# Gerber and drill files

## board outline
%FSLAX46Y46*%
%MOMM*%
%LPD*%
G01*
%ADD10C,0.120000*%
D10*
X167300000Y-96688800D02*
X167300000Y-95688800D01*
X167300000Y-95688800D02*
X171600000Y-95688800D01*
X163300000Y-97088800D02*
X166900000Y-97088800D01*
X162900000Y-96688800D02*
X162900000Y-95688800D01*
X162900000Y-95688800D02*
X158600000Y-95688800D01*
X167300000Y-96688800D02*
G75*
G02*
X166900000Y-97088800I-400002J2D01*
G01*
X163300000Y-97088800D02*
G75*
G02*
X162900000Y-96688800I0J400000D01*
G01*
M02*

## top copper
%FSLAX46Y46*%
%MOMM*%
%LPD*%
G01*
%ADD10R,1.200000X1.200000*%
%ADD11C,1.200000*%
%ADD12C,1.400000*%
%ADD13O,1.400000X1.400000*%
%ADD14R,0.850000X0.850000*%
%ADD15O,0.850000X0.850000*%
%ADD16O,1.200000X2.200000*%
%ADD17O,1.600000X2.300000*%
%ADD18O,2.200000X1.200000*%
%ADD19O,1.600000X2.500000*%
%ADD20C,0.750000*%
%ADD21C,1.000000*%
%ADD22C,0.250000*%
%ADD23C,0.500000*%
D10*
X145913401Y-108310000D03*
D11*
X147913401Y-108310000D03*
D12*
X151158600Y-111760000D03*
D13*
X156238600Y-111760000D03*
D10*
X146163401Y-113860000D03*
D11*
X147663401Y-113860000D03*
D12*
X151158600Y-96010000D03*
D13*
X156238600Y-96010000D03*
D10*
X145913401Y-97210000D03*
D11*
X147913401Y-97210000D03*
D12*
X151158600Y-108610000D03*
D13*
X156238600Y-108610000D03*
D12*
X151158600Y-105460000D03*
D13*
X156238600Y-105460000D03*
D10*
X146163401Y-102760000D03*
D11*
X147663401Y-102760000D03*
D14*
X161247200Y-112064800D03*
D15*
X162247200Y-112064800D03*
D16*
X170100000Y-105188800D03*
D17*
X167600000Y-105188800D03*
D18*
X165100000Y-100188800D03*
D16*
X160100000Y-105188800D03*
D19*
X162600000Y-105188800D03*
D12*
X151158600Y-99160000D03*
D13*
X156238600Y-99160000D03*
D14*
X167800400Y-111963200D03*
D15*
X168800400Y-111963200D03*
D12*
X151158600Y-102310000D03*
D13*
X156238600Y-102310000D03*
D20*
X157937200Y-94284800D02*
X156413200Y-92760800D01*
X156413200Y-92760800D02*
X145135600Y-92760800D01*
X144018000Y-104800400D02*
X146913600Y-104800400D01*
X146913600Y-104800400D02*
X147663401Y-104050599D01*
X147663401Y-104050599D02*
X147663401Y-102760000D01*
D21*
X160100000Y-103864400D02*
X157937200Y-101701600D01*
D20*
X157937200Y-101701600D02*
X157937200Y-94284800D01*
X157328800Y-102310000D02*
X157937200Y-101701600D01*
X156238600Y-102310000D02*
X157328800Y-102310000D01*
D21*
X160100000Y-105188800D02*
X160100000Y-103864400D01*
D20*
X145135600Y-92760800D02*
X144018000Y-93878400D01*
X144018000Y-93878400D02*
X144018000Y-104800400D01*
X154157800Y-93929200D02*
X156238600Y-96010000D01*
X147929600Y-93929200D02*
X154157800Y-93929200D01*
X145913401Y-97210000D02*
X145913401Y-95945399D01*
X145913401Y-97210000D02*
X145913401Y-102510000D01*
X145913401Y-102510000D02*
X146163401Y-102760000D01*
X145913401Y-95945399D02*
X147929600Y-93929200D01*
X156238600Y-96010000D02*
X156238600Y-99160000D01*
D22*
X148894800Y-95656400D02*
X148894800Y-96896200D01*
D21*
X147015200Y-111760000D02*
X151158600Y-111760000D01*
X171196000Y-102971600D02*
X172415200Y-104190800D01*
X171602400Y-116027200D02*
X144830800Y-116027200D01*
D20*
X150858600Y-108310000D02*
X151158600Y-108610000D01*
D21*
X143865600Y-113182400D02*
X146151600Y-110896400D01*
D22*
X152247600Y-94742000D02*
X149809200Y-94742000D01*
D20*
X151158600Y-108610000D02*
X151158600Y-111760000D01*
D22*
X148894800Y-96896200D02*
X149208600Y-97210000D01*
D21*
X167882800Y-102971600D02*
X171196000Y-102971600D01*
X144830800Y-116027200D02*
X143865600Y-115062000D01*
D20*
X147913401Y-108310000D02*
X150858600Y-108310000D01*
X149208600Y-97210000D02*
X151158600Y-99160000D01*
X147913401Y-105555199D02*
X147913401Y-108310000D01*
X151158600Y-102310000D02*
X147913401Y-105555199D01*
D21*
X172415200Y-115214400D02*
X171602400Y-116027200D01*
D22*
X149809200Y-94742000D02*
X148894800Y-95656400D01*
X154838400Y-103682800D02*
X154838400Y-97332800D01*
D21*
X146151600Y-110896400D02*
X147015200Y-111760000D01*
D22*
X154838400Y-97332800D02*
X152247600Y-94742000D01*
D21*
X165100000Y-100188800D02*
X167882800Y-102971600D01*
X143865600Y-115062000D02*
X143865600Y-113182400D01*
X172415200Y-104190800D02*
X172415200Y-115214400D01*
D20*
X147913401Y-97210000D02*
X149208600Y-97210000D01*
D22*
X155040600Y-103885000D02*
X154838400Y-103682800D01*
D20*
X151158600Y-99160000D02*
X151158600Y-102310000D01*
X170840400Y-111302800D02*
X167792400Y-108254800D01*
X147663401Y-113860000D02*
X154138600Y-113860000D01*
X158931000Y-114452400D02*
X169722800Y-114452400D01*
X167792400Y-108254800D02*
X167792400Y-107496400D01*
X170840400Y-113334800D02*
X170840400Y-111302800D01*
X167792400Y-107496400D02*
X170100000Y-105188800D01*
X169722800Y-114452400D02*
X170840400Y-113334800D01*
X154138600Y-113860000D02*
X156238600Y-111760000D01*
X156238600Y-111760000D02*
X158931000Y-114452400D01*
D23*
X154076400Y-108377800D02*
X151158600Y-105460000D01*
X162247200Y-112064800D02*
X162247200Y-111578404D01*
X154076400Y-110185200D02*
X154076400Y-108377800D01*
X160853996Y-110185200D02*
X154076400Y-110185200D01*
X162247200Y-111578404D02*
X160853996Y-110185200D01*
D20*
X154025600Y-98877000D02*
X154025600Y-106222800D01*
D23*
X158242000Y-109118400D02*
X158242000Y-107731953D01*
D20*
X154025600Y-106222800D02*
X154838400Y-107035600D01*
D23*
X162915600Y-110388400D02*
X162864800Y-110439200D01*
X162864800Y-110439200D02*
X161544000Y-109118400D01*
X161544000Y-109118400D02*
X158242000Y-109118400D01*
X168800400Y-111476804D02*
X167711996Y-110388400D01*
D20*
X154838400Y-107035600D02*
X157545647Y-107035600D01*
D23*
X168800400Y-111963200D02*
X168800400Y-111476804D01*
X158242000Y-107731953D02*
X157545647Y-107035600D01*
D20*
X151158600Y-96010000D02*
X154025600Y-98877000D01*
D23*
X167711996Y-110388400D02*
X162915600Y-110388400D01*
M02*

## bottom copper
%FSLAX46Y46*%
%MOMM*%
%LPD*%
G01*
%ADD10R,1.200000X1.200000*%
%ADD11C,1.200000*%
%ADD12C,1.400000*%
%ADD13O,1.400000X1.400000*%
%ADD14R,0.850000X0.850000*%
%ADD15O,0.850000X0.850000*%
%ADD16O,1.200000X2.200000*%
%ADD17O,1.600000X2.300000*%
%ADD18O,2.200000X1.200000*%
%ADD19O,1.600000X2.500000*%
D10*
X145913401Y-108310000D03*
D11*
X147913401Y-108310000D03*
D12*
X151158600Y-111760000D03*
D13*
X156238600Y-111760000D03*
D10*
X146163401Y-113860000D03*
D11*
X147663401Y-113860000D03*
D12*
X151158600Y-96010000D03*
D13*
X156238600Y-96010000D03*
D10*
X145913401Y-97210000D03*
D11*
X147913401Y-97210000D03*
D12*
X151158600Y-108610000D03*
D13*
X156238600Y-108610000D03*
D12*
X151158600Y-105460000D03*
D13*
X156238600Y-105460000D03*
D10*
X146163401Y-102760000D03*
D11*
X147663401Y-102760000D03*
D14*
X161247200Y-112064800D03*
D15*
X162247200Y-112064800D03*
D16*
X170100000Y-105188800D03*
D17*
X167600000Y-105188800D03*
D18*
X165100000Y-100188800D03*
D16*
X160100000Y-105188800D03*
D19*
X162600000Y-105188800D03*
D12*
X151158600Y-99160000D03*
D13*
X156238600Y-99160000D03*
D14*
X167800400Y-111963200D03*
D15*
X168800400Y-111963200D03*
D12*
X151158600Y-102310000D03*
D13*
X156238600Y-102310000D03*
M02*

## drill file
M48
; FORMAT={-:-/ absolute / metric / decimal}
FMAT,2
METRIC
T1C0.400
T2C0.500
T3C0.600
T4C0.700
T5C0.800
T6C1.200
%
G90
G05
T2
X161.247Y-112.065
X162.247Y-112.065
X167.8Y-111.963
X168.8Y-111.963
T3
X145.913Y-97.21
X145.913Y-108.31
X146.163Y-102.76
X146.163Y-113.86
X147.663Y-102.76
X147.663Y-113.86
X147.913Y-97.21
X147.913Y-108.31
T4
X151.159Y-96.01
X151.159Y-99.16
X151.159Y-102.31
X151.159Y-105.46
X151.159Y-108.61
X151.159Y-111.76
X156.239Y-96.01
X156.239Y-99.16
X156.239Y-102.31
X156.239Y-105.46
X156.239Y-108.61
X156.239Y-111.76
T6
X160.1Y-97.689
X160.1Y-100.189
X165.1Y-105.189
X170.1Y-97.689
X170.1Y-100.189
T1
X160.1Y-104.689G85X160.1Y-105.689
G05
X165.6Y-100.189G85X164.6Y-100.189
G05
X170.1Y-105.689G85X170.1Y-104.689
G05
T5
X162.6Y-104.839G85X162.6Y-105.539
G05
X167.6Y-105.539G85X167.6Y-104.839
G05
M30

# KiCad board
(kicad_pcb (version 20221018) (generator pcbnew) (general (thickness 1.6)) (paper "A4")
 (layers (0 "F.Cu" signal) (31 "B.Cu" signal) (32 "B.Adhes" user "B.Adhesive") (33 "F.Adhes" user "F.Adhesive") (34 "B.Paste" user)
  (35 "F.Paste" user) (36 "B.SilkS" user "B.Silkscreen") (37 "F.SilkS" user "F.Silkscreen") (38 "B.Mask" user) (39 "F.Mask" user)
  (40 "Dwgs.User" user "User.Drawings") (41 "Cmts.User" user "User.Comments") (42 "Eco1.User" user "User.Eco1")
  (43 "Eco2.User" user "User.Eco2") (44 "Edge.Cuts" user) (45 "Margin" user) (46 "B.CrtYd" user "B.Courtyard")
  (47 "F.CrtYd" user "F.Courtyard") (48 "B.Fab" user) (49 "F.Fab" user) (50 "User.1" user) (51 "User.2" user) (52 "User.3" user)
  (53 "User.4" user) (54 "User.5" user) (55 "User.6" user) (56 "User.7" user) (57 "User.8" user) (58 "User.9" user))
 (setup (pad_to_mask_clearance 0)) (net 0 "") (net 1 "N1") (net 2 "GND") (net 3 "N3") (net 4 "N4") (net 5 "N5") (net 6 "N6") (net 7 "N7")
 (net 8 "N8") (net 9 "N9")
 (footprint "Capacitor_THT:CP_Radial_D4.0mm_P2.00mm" (layer "F.Cu") (at 145.913401 108.31)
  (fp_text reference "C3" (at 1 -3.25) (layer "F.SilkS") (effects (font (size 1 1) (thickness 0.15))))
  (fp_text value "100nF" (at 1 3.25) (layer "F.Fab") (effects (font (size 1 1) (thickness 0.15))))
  (pad "1" thru_hole rect (at 0 0) (size 1.2 1.2) (drill 0.6) (layers "*.Cu" "*.Mask") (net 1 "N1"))
  (pad "2" thru_hole circle (at 2 0) (size 1.2 1.2) (drill 0.6) (layers "*.Cu" "*.Mask") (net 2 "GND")))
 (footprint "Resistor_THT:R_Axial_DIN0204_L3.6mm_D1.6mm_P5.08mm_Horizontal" (layer "F.Cu") (at 151.1586 111.76)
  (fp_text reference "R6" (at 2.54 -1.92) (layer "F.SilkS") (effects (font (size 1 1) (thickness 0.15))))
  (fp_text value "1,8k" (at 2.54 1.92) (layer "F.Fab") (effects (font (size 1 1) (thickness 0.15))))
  (pad "1" thru_hole circle (at 0 0) (size 1.4 1.4) (drill 0.7) (layers "*.Cu" "*.Mask") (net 2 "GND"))
  (pad "2" thru_hole oval (at 5.08 0) (size 1.4 1.4) (drill 0.7) (layers "*.Cu" "*.Mask") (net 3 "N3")))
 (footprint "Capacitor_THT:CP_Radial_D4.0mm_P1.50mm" (layer "F.Cu") (at 146.163401 113.86)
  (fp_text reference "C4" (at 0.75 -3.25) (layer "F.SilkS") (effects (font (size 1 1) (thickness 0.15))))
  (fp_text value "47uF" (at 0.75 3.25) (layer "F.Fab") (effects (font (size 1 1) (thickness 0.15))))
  (pad "1" thru_hole rect (at 0 0) (size 1.2 1.2) (drill 0.6) (layers "*.Cu" "*.Mask") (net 1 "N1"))
  (pad "2" thru_hole circle (at 1.5 0) (size 1.2 1.2) (drill 0.6) (layers "*.Cu" "*.Mask") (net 3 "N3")))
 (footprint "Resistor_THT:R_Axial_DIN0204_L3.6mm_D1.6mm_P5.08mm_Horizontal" (layer "F.Cu") (at 151.1586 96.01)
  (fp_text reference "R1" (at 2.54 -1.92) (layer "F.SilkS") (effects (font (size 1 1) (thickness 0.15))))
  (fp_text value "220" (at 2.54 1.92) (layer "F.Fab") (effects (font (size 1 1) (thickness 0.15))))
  (pad "1" thru_hole circle (at 0 0) (size 1.4 1.4) (drill 0.7) (layers "*.Cu" "*.Mask") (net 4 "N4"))
  (pad "2" thru_hole oval (at 5.08 0) (size 1.4 1.4) (drill 0.7) (layers "*.Cu" "*.Mask") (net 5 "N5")))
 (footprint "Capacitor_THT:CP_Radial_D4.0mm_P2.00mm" (layer "F.Cu") (at 145.913401 97.21)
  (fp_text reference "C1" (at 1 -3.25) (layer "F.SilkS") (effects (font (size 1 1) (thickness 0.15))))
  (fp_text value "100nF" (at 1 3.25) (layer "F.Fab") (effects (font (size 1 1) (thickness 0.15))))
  (pad "1" thru_hole rect (at 0 0) (size 1.2 1.2) (drill 0.6) (layers "*.Cu" "*.Mask") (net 5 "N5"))
  (pad "2" thru_hole circle (at 2 0) (size 1.2 1.2) (drill 0.6) (layers "*.Cu" "*.Mask") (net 2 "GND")))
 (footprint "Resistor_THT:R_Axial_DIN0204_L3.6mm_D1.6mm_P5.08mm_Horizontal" (layer "F.Cu") (at 151.1586 108.61)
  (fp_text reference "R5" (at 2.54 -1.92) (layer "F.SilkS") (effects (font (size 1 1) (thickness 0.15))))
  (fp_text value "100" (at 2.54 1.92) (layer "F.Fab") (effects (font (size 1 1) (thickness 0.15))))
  (pad "1" thru_hole circle (at 0 0) (size 1.4 1.4) (drill 0.7) (layers "*.Cu" "*.Mask") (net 2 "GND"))
  (pad "2" thru_hole oval (at 5.08 0) (size 1.4 1.4) (drill 0.7) (layers "*.Cu" "*.Mask") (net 1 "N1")))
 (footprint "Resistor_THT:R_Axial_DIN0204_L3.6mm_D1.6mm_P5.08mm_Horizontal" (layer "F.Cu") (at 151.1586 105.46)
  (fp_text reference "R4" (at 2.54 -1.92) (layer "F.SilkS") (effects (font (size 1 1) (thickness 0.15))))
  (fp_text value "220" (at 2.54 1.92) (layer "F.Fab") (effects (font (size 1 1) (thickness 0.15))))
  (pad "1" thru_hole circle (at 0 0) (size 1.4 1.4) (drill 0.7) (layers "*.Cu" "*.Mask") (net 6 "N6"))
  (pad "2" thru_hole oval (at 5.08 0) (size 1.4 1.4) (drill 0.7) (layers "*.Cu" "*.Mask") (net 1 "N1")))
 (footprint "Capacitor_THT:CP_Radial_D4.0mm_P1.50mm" (layer "F.Cu") (at 146.163401 102.76)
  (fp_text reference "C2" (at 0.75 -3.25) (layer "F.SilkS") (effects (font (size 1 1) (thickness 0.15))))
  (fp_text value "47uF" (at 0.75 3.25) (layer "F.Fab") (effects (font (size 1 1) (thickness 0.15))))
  (pad "1" thru_hole rect (at 0 0) (size 1.2 1.2) (drill 0.6) (layers "*.Cu" "*.Mask") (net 5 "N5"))
  (pad "2" thru_hole circle (at 1.5 0) (size 1.2 1.2) (drill 0.6) (layers "*.Cu" "*.Mask") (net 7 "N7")))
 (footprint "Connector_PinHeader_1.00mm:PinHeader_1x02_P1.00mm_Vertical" (layer "F.Cu") (at 161.2472 112.0648 90)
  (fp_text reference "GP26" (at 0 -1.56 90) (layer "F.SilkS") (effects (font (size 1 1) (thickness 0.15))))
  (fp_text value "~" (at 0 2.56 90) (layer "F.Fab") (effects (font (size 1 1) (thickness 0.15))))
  (pad "1" thru_hole rect (at 0 0 90) (size 0.85 0.85) (drill 0.5) (layers "*.Cu" "*.Mask") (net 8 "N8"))
  (pad "2" thru_hole oval (at 0 1 90) (size 0.85 0.85) (drill 0.5) (layers "*.Cu" "*.Mask") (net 6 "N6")))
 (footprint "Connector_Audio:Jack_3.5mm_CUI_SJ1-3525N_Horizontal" (layer "F.Cu") (at 165.1 100.1888 180)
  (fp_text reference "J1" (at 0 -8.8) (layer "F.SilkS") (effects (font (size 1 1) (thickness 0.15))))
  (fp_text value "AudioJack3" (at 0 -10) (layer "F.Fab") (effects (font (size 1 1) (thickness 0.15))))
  (fp_line (start -2.2 3.5) (end -2.2 4.5) (stroke (width 0.12) (type solid)) (layer "Edge.Cuts"))
  (fp_line (start -2.2 4.5) (end -6.5 4.5) (stroke (width 0.12) (type solid)) (layer "Edge.Cuts"))
  (fp_line (start 1.8 3.1) (end -1.8 3.1) (stroke (width 0.12) (type solid)) (layer "Edge.Cuts"))
  (fp_line (start 2.2 3.5) (end 2.2 4.5) (stroke (width 0.12) (type solid)) (layer "Edge.Cuts"))
  (fp_line (start 2.2 4.5) (end 6.5 4.5) (stroke (width 0.12) (type solid)) (layer "Edge.Cuts"))
  (fp_arc (start -2.2 3.5) (mid -2.082842 3.217158) (end -1.8 3.1) (stroke (width 0.12) (type solid)) (layer "Edge.Cuts"))
  (fp_arc (start 1.8 3.1) (mid 2.082843 3.217157) (end 2.2 3.5) (stroke (width 0.12) (type solid)) (layer "Edge.Cuts"))
  (pad "" np_thru_hole circle (at -5 0 180) (size 1.2 1.2) (drill 1.2) (layers "*.Cu"))
  (pad "" np_thru_hole circle (at -5 2.5 180) (size 1.2 1.2) (drill 1.2) (layers "*.Cu"))
  (pad "" np_thru_hole circle (at 0 -5 180) (size 1.2 1.2) (drill 1.2) (layers "*.Cu"))
  (pad "" np_thru_hole circle (at 5 0 180) (size 1.2 1.2) (drill 1.2) (layers "*.Cu"))
  (pad "" np_thru_hole circle (at 5 2.5 180) (size 1.2 1.2) (drill 1.2) (layers "*.Cu"))
  (pad "R" thru_hole oval (at -5 -5 180) (size 1.2 2.2) (drill oval 0.4 1.4) (layers "*.Cu" "*.Mask") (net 3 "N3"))
  (pad "RN" thru_hole oval (at -2.5 -5 180) (size 1.6 2.3) (drill oval 0.8 1.5) (layers "*.Cu" "*.Mask"))
  (pad "S" thru_hole oval (at 0 0 180) (size 2.2 1.2) (drill oval 1.4 0.4) (layers "*.Cu" "*.Mask") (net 2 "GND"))
  (pad "T" thru_hole oval (at 5 -5) (size 1.2 2.2) (drill oval 0.4 1.4) (layers "*.Cu" "*.Mask") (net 7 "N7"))
  (pad "TN" thru_hole oval (at 2.5 -5) (size 1.6 2.5) (drill oval 0.8 1.5) (layers "*.Cu" "*.Mask")))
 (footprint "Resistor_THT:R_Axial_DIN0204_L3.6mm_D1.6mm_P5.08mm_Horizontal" (layer "F.Cu") (at 151.1586 99.16)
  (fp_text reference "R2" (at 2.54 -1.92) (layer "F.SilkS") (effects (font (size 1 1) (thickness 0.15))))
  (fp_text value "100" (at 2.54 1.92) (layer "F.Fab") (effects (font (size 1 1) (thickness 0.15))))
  (pad "1" thru_hole circle (at 0 0) (size 1.4 1.4) (drill 0.7) (layers "*.Cu" "*.Mask") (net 2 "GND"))
  (pad "2" thru_hole oval (at 5.08 0) (size 1.4 1.4) (drill 0.7) (layers "*.Cu" "*.Mask") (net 5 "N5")))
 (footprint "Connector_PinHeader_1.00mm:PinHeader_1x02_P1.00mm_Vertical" (layer "F.Cu") (at 167.8004 111.9632 90)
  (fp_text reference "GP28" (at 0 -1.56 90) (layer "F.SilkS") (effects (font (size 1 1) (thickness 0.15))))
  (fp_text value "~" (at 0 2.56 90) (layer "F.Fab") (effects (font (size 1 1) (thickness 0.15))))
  (pad "1" thru_hole rect (at 0 0 90) (size 0.85 0.85) (drill 0.5) (layers "*.Cu" "*.Mask") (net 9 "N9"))
  (pad "2" thru_hole oval (at 0 1 90) (size 0.85 0.85) (drill 0.5) (layers "*.Cu" "*.Mask") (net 4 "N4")))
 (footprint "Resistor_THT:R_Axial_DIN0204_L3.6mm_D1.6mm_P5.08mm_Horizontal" (layer "F.Cu") (at 151.1586 102.31)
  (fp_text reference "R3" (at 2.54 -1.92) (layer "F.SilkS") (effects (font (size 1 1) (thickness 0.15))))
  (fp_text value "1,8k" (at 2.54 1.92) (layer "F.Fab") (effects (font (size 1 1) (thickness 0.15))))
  (pad "1" thru_hole circle (at 0 0) (size 1.4 1.4) (drill 0.7) (layers "*.Cu" "*.Mask") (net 2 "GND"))
  (pad "2" thru_hole oval (at 5.08 0) (size 1.4 1.4) (drill 0.7) (layers "*.Cu" "*.Mask") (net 7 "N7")))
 (segment (start 157.9372 94.2848) (end 156.4132 92.7608) (width 0.75) (layer "F.Cu") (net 7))
 (segment (start 156.4132 92.7608) (end 145.1356 92.7608) (width 0.75) (layer "F.Cu") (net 7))
 (segment (start 144.018 104.8004) (end 146.9136 104.8004) (width 0.75) (layer "F.Cu") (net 7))
 (segment (start 146.9136 104.8004) (end 147.663401 104.050599) (width 0.75) (layer "F.Cu") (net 7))
 (segment (start 147.663401 104.050599) (end 147.663401 102.76) (width 0.75) (layer "F.Cu") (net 7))
 (segment (start 160.1 103.8644) (end 157.9372 101.7016) (width 1) (layer "F.Cu") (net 7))
 (segment (start 157.9372 101.7016) (end 157.9372 94.2848) (width 0.75) (layer "F.Cu") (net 7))
 (segment (start 157.3288 102.31) (end 157.9372 101.7016) (width 0.75) (layer "F.Cu") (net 7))
 (segment (start 156.2386 102.31) (end 157.3288 102.31) (width 0.75) (layer "F.Cu") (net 7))
 (segment (start 160.1 105.1888) (end 160.1 103.8644) (width 1) (layer "F.Cu") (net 7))
 (segment (start 145.1356 92.7608) (end 144.018 93.8784) (width 0.75) (layer "F.Cu") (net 7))
 (segment (start 144.018 93.8784) (end 144.018 104.8004) (width 0.75) (layer "F.Cu") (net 7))
 (segment (start 154.1578 93.9292) (end 156.2386 96.01) (width 0.75) (layer "F.Cu") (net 5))
 (segment (start 147.9296 93.9292) (end 154.1578 93.9292) (width 0.75) (layer "F.Cu") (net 5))
 (segment (start 145.913401 97.21) (end 145.913401 95.945399) (width 0.75) (layer "F.Cu") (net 5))
 (segment (start 145.913401 97.21) (end 145.913401 102.51) (width 0.75) (layer "F.Cu") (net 5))
 (segment (start 145.913401 102.51) (end 146.163401 102.76) (width 0.75) (layer "F.Cu") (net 5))
 (segment (start 145.913401 95.945399) (end 147.9296 93.9292) (width 0.75) (layer "F.Cu") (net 5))
 (segment (start 156.2386 96.01) (end 156.2386 99.16) (width 0.75) (layer "F.Cu") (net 5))
 (segment (start 148.8948 95.6564) (end 148.8948 96.8962) (width 0.25) (layer "F.Cu") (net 2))
 (segment (start 147.0152 111.76) (end 151.1586 111.76) (width 1) (layer "F.Cu") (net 2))
 (segment (start 171.196 102.9716) (end 172.4152 104.1908) (width 1) (layer "F.Cu") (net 2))
 (segment (start 171.6024 116.0272) (end 144.8308 116.0272) (width 1) (layer "F.Cu") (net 2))
 (segment (start 150.8586 108.31) (end 151.1586 108.61) (width 0.75) (layer "F.Cu") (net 2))
 (segment (start 143.8656 113.1824) (end 146.1516 110.8964) (width 1) (layer "F.Cu") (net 2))
 (segment (start 152.2476 94.742) (end 149.8092 94.742) (width 0.25) (layer "F.Cu") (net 2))
 (segment (start 151.1586 108.61) (end 151.1586 111.76) (width 0.75) (layer "F.Cu") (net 2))
 (segment (start 148.8948 96.8962) (end 149.2086 97.21) (width 0.25) (layer "F.Cu") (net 2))
 (segment (start 167.8828 102.9716) (end 171.196 102.9716) (width 1) (layer "F.Cu") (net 2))
 (segment (start 144.8308 116.0272) (end 143.8656 115.062) (width 1) (layer "F.Cu") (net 2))
 (segment (start 147.913401 108.31) (end 150.8586 108.31) (width 0.75) (layer "F.Cu") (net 2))
 (segment (start 149.2086 97.21) (end 151.1586 99.16) (width 0.75) (layer "F.Cu") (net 2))
 (segment (start 147.913401 105.555199) (end 147.913401 108.31) (width 0.75) (layer "F.Cu") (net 2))
 (segment (start 151.1586 102.31) (end 147.913401 105.555199) (width 0.75) (layer "F.Cu") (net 2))
 (segment (start 172.4152 115.2144) (end 171.6024 116.0272) (width 1) (layer "F.Cu") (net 2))
 (segment (start 149.8092 94.742) (end 148.8948 95.6564) (width 0.25) (layer "F.Cu") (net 2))
 (segment (start 154.8384 103.6828) (end 154.8384 97.3328) (width 0.25) (layer "F.Cu") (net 2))
 (segment (start 146.1516 110.8964) (end 147.0152 111.76) (width 1) (layer "F.Cu") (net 2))
 (segment (start 154.8384 97.3328) (end 152.2476 94.742) (width 0.25) (layer "F.Cu") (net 2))
 (segment (start 165.1 100.1888) (end 167.8828 102.9716) (width 1) (layer "F.Cu") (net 2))
 (segment (start 143.8656 115.062) (end 143.8656 113.1824) (width 1) (layer "F.Cu") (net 2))
 (segment (start 172.4152 104.1908) (end 172.4152 115.2144) (width 1) (layer "F.Cu") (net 2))
 (segment (start 147.913401 97.21) (end 149.2086 97.21) (width 0.75) (layer "F.Cu") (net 2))
 (segment (start 155.0406 103.885) (end 154.8384 103.6828) (width 0.25) (layer "F.Cu") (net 2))
 (segment (start 151.1586 99.16) (end 151.1586 102.31) (width 0.75) (layer "F.Cu") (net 2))
 (segment (start 170.8404 111.3028) (end 167.7924 108.2548) (width 0.75) (layer "F.Cu") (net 3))
 (segment (start 147.663401 113.86) (end 154.1386 113.86) (width 0.75) (layer "F.Cu") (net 3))
 (segment (start 158.931 114.4524) (end 169.7228 114.4524) (width 0.75) (layer "F.Cu") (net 3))
 (segment (start 167.7924 108.2548) (end 167.7924 107.4964) (width 0.75) (layer "F.Cu") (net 3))
 (segment (start 170.8404 113.3348) (end 170.8404 111.3028) (width 0.75) (layer "F.Cu") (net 3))
 (segment (start 167.7924 107.4964) (end 170.1 105.1888) (width 0.75) (layer "F.Cu") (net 3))
 (segment (start 169.7228 114.4524) (end 170.8404 113.3348) (width 0.75) (layer "F.Cu") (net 3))
 (segment (start 154.1386 113.86) (end 156.2386 111.76) (width 0.75) (layer "F.Cu") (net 3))
 (segment (start 156.2386 111.76) (end 158.931 114.4524) (width 0.75) (layer "F.Cu") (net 3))
 (segment (start 154.0764 108.3778) (end 151.1586 105.46) (width 0.5) (layer "F.Cu") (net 6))
 (segment (start 162.2472 112.0648) (end 162.2472 111.578404) (width 0.5) (layer "F.Cu") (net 6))
 (segment (start 154.0764 110.1852) (end 154.0764 108.3778) (width 0.5) (layer "F.Cu") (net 6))
 (segment (start 160.853996 110.1852) (end 154.0764 110.1852) (width 0.5) (layer "F.Cu") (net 6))
 (segment (start 162.2472 111.578404) (end 160.853996 110.1852) (width 0.5) (layer "F.Cu") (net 6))
 (segment (start 154.0256 98.877) (end 154.0256 106.2228) (width 0.75) (layer "F.Cu") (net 4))
 (segment (start 158.242 109.1184) (end 158.242 107.731953) (width 0.5) (layer "F.Cu") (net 4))
 (segment (start 154.0256 106.2228) (end 154.8384 107.0356) (width 0.75) (layer "F.Cu") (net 4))
 (segment (start 162.9156 110.3884) (end 162.8648 110.4392) (width 0.5) (layer "F.Cu") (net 4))
 (segment (start 162.8648 110.4392) (end 161.544 109.1184) (width 0.5) (layer "F.Cu") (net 4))
 (segment (start 161.544 109.1184) (end 158.242 109.1184) (width 0.5) (layer "F.Cu") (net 4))
 (segment (start 168.8004 111.476804) (end 167.711996 110.3884) (width 0.5) (layer "F.Cu") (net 4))
 (segment (start 154.8384 107.0356) (end 157.545647 107.0356) (width 0.75) (layer "F.Cu") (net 4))
 (segment (start 168.8004 111.9632) (end 168.8004 111.476804) (width 0.5) (layer "F.Cu") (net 4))
 (segment (start 158.242 107.731953) (end 157.545647 107.0356) (width 0.5) (layer "F.Cu") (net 4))
 (segment (start 151.1586 96.01) (end 154.0256 98.877) (width 0.75) (layer "F.Cu") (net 4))
 (segment (start 167.711996 110.3884) (end 162.9156 110.3884) (width 0.5) (layer "F.Cu") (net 4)))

